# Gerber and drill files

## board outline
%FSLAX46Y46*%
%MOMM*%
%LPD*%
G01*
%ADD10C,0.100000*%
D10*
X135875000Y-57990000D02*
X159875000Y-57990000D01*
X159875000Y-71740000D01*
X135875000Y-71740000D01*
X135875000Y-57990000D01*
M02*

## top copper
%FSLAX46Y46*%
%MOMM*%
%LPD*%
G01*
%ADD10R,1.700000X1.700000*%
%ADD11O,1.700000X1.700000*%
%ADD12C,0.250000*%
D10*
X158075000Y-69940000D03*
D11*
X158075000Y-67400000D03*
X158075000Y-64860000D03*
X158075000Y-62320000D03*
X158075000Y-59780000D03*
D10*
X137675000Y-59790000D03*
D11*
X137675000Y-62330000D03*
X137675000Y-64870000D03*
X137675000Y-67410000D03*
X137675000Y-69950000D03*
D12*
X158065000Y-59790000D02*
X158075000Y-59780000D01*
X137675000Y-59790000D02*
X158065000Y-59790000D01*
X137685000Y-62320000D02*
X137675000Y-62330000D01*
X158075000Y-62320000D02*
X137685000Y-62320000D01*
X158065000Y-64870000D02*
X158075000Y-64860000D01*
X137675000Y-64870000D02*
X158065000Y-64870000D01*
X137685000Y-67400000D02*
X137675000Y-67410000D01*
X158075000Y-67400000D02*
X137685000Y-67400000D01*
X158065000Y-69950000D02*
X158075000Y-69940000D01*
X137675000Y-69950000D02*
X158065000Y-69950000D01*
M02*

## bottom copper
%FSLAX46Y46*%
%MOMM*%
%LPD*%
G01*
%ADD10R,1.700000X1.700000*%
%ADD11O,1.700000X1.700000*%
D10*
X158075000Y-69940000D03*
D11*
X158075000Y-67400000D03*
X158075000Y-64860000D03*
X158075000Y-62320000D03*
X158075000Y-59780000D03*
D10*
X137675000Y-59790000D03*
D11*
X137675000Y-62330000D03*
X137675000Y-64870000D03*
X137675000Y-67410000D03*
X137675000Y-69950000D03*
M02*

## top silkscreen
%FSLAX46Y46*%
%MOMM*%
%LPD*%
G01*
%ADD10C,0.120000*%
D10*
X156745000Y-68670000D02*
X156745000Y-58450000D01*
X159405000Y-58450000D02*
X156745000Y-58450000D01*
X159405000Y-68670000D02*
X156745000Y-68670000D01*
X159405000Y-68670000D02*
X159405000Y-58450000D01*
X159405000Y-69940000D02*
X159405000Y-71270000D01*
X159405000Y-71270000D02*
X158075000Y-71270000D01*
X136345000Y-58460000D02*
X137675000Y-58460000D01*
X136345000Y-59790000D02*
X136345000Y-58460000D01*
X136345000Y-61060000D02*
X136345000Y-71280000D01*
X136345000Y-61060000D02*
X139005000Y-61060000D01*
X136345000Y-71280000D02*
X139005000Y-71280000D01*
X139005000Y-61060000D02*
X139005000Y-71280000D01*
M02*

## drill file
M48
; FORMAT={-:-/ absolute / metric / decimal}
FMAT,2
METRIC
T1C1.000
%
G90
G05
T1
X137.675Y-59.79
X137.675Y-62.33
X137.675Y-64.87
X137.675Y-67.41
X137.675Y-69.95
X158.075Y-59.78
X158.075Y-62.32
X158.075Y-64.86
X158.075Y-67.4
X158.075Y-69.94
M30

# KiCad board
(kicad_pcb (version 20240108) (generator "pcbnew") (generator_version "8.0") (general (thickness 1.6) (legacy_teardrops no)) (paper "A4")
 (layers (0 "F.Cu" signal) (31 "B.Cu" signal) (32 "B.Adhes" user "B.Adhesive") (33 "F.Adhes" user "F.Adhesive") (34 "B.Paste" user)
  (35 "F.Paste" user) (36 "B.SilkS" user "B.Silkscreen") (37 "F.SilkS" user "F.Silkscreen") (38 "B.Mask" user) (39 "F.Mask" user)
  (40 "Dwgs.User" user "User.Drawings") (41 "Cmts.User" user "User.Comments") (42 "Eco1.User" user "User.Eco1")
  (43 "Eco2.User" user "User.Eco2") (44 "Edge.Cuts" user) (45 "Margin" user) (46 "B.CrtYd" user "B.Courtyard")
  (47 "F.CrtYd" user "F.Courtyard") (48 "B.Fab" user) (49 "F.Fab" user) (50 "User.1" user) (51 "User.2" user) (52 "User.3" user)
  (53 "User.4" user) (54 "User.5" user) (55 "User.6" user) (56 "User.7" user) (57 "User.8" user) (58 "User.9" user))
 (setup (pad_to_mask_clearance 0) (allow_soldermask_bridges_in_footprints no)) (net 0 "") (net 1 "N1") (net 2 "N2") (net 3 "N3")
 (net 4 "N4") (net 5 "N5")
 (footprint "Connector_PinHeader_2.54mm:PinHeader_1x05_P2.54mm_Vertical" (layer "F.Cu") (at 158.075 69.94 180)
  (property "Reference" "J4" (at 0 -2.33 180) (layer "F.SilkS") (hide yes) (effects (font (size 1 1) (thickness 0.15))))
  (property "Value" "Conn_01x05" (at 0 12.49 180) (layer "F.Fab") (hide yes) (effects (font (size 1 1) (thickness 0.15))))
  (fp_line (start 1.33 1.27) (end 1.33 11.49) (stroke (width 0.12) (type solid)) (layer "F.SilkS"))
  (fp_line (start -1.33 11.49) (end 1.33 11.49) (stroke (width 0.12) (type solid)) (layer "F.SilkS"))
  (fp_line (start -1.33 1.27) (end 1.33 1.27) (stroke (width 0.12) (type solid)) (layer "F.SilkS"))
  (fp_line (start -1.33 1.27) (end -1.33 11.49) (stroke (width 0.12) (type solid)) (layer "F.SilkS"))
  (fp_line (start -1.33 0) (end -1.33 -1.33) (stroke (width 0.12) (type solid)) (layer "F.SilkS"))
  (fp_line (start -1.33 -1.33) (end 0 -1.33) (stroke (width 0.12) (type solid)) (layer "F.SilkS"))
  (pad "1" thru_hole rect (at 0 0 180) (size 1.7 1.7) (drill 1) (layers "*.Cu" "*.Mask") (remove_unused_layers no) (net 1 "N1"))
  (pad "2" thru_hole oval (at 0 2.54 180) (size 1.7 1.7) (drill 1) (layers "*.Cu" "*.Mask") (remove_unused_layers no) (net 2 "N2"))
  (pad "3" thru_hole oval (at 0 5.08 180) (size 1.7 1.7) (drill 1) (layers "*.Cu" "*.Mask") (remove_unused_layers no) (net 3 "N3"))
  (pad "4" thru_hole oval (at 0 7.62 180) (size 1.7 1.7) (drill 1) (layers "*.Cu" "*.Mask") (remove_unused_layers no) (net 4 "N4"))
  (pad "5" thru_hole oval (at 0 10.16 180) (size 1.7 1.7) (drill 1) (layers "*.Cu" "*.Mask") (remove_unused_layers no) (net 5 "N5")))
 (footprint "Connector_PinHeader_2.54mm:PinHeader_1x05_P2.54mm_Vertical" (layer "F.Cu") (at 137.675 59.79)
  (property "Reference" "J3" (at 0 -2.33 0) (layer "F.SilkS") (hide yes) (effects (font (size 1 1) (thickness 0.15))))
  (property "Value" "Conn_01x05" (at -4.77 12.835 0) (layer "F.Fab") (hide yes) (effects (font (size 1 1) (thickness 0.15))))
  (fp_line (start -1.33 -1.33) (end 0 -1.33) (stroke (width 0.12) (type solid)) (layer "F.SilkS"))
  (fp_line (start -1.33 0) (end -1.33 -1.33) (stroke (width 0.12) (type solid)) (layer "F.SilkS"))
  (fp_line (start -1.33 1.27) (end -1.33 11.49) (stroke (width 0.12) (type solid)) (layer "F.SilkS"))
  (fp_line (start -1.33 1.27) (end 1.33 1.27) (stroke (width 0.12) (type solid)) (layer "F.SilkS"))
  (fp_line (start -1.33 11.49) (end 1.33 11.49) (stroke (width 0.12) (type solid)) (layer "F.SilkS"))
  (fp_line (start 1.33 1.27) (end 1.33 11.49) (stroke (width 0.12) (type solid)) (layer "F.SilkS"))
  (pad "1" thru_hole rect (at 0 0) (size 1.7 1.7) (drill 1) (layers "*.Cu" "*.Mask") (remove_unused_layers no) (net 5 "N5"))
  (pad "2" thru_hole oval (at 0 2.54) (size 1.7 1.7) (drill 1) (layers "*.Cu" "*.Mask") (remove_unused_layers no) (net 4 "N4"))
  (pad "3" thru_hole oval (at 0 5.08) (size 1.7 1.7) (drill 1) (layers "*.Cu" "*.Mask") (remove_unused_layers no) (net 3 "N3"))
  (pad "4" thru_hole oval (at 0 7.62) (size 1.7 1.7) (drill 1) (layers "*.Cu" "*.Mask") (remove_unused_layers no) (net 2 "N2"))
  (pad "5" thru_hole oval (at 0 10.16) (size 1.7 1.7) (drill 1) (layers "*.Cu" "*.Mask") (remove_unused_layers no) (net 1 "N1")))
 (gr_rect (start 135.875 57.99) (end 159.875 71.74) (stroke (width 0.1) (type default)) (fill none) (layer "Edge.Cuts"))
 (segment (start 158.065 59.79) (end 158.075 59.78) (width 0.25) (layer "F.Cu") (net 5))
 (segment (start 137.675 59.79) (end 158.065 59.79) (width 0.25) (layer "F.Cu") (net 5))
 (segment (start 137.685 62.32) (end 137.675 62.33) (width 0.25) (layer "F.Cu") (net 4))
 (segment (start 158.075 62.32) (end 137.685 62.32) (width 0.25) (layer "F.Cu") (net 4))
 (segment (start 158.065 64.87) (end 158.075 64.86) (width 0.25) (layer "F.Cu") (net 3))
 (segment (start 137.675 64.87) (end 158.065 64.87) (width 0.25) (layer "F.Cu") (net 3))
 (segment (start 137.685 67.4) (end 137.675 67.41) (width 0.25) (layer "F.Cu") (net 2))
 (segment (start 158.075 67.4) (end 137.685 67.4) (width 0.25) (layer "F.Cu") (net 2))
 (segment (start 158.065 69.95) (end 158.075 69.94) (width 0.25) (layer "F.Cu") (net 1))
 (segment (start 137.675 69.95) (end 158.065 69.95) (width 0.25) (layer "F.Cu") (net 1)))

